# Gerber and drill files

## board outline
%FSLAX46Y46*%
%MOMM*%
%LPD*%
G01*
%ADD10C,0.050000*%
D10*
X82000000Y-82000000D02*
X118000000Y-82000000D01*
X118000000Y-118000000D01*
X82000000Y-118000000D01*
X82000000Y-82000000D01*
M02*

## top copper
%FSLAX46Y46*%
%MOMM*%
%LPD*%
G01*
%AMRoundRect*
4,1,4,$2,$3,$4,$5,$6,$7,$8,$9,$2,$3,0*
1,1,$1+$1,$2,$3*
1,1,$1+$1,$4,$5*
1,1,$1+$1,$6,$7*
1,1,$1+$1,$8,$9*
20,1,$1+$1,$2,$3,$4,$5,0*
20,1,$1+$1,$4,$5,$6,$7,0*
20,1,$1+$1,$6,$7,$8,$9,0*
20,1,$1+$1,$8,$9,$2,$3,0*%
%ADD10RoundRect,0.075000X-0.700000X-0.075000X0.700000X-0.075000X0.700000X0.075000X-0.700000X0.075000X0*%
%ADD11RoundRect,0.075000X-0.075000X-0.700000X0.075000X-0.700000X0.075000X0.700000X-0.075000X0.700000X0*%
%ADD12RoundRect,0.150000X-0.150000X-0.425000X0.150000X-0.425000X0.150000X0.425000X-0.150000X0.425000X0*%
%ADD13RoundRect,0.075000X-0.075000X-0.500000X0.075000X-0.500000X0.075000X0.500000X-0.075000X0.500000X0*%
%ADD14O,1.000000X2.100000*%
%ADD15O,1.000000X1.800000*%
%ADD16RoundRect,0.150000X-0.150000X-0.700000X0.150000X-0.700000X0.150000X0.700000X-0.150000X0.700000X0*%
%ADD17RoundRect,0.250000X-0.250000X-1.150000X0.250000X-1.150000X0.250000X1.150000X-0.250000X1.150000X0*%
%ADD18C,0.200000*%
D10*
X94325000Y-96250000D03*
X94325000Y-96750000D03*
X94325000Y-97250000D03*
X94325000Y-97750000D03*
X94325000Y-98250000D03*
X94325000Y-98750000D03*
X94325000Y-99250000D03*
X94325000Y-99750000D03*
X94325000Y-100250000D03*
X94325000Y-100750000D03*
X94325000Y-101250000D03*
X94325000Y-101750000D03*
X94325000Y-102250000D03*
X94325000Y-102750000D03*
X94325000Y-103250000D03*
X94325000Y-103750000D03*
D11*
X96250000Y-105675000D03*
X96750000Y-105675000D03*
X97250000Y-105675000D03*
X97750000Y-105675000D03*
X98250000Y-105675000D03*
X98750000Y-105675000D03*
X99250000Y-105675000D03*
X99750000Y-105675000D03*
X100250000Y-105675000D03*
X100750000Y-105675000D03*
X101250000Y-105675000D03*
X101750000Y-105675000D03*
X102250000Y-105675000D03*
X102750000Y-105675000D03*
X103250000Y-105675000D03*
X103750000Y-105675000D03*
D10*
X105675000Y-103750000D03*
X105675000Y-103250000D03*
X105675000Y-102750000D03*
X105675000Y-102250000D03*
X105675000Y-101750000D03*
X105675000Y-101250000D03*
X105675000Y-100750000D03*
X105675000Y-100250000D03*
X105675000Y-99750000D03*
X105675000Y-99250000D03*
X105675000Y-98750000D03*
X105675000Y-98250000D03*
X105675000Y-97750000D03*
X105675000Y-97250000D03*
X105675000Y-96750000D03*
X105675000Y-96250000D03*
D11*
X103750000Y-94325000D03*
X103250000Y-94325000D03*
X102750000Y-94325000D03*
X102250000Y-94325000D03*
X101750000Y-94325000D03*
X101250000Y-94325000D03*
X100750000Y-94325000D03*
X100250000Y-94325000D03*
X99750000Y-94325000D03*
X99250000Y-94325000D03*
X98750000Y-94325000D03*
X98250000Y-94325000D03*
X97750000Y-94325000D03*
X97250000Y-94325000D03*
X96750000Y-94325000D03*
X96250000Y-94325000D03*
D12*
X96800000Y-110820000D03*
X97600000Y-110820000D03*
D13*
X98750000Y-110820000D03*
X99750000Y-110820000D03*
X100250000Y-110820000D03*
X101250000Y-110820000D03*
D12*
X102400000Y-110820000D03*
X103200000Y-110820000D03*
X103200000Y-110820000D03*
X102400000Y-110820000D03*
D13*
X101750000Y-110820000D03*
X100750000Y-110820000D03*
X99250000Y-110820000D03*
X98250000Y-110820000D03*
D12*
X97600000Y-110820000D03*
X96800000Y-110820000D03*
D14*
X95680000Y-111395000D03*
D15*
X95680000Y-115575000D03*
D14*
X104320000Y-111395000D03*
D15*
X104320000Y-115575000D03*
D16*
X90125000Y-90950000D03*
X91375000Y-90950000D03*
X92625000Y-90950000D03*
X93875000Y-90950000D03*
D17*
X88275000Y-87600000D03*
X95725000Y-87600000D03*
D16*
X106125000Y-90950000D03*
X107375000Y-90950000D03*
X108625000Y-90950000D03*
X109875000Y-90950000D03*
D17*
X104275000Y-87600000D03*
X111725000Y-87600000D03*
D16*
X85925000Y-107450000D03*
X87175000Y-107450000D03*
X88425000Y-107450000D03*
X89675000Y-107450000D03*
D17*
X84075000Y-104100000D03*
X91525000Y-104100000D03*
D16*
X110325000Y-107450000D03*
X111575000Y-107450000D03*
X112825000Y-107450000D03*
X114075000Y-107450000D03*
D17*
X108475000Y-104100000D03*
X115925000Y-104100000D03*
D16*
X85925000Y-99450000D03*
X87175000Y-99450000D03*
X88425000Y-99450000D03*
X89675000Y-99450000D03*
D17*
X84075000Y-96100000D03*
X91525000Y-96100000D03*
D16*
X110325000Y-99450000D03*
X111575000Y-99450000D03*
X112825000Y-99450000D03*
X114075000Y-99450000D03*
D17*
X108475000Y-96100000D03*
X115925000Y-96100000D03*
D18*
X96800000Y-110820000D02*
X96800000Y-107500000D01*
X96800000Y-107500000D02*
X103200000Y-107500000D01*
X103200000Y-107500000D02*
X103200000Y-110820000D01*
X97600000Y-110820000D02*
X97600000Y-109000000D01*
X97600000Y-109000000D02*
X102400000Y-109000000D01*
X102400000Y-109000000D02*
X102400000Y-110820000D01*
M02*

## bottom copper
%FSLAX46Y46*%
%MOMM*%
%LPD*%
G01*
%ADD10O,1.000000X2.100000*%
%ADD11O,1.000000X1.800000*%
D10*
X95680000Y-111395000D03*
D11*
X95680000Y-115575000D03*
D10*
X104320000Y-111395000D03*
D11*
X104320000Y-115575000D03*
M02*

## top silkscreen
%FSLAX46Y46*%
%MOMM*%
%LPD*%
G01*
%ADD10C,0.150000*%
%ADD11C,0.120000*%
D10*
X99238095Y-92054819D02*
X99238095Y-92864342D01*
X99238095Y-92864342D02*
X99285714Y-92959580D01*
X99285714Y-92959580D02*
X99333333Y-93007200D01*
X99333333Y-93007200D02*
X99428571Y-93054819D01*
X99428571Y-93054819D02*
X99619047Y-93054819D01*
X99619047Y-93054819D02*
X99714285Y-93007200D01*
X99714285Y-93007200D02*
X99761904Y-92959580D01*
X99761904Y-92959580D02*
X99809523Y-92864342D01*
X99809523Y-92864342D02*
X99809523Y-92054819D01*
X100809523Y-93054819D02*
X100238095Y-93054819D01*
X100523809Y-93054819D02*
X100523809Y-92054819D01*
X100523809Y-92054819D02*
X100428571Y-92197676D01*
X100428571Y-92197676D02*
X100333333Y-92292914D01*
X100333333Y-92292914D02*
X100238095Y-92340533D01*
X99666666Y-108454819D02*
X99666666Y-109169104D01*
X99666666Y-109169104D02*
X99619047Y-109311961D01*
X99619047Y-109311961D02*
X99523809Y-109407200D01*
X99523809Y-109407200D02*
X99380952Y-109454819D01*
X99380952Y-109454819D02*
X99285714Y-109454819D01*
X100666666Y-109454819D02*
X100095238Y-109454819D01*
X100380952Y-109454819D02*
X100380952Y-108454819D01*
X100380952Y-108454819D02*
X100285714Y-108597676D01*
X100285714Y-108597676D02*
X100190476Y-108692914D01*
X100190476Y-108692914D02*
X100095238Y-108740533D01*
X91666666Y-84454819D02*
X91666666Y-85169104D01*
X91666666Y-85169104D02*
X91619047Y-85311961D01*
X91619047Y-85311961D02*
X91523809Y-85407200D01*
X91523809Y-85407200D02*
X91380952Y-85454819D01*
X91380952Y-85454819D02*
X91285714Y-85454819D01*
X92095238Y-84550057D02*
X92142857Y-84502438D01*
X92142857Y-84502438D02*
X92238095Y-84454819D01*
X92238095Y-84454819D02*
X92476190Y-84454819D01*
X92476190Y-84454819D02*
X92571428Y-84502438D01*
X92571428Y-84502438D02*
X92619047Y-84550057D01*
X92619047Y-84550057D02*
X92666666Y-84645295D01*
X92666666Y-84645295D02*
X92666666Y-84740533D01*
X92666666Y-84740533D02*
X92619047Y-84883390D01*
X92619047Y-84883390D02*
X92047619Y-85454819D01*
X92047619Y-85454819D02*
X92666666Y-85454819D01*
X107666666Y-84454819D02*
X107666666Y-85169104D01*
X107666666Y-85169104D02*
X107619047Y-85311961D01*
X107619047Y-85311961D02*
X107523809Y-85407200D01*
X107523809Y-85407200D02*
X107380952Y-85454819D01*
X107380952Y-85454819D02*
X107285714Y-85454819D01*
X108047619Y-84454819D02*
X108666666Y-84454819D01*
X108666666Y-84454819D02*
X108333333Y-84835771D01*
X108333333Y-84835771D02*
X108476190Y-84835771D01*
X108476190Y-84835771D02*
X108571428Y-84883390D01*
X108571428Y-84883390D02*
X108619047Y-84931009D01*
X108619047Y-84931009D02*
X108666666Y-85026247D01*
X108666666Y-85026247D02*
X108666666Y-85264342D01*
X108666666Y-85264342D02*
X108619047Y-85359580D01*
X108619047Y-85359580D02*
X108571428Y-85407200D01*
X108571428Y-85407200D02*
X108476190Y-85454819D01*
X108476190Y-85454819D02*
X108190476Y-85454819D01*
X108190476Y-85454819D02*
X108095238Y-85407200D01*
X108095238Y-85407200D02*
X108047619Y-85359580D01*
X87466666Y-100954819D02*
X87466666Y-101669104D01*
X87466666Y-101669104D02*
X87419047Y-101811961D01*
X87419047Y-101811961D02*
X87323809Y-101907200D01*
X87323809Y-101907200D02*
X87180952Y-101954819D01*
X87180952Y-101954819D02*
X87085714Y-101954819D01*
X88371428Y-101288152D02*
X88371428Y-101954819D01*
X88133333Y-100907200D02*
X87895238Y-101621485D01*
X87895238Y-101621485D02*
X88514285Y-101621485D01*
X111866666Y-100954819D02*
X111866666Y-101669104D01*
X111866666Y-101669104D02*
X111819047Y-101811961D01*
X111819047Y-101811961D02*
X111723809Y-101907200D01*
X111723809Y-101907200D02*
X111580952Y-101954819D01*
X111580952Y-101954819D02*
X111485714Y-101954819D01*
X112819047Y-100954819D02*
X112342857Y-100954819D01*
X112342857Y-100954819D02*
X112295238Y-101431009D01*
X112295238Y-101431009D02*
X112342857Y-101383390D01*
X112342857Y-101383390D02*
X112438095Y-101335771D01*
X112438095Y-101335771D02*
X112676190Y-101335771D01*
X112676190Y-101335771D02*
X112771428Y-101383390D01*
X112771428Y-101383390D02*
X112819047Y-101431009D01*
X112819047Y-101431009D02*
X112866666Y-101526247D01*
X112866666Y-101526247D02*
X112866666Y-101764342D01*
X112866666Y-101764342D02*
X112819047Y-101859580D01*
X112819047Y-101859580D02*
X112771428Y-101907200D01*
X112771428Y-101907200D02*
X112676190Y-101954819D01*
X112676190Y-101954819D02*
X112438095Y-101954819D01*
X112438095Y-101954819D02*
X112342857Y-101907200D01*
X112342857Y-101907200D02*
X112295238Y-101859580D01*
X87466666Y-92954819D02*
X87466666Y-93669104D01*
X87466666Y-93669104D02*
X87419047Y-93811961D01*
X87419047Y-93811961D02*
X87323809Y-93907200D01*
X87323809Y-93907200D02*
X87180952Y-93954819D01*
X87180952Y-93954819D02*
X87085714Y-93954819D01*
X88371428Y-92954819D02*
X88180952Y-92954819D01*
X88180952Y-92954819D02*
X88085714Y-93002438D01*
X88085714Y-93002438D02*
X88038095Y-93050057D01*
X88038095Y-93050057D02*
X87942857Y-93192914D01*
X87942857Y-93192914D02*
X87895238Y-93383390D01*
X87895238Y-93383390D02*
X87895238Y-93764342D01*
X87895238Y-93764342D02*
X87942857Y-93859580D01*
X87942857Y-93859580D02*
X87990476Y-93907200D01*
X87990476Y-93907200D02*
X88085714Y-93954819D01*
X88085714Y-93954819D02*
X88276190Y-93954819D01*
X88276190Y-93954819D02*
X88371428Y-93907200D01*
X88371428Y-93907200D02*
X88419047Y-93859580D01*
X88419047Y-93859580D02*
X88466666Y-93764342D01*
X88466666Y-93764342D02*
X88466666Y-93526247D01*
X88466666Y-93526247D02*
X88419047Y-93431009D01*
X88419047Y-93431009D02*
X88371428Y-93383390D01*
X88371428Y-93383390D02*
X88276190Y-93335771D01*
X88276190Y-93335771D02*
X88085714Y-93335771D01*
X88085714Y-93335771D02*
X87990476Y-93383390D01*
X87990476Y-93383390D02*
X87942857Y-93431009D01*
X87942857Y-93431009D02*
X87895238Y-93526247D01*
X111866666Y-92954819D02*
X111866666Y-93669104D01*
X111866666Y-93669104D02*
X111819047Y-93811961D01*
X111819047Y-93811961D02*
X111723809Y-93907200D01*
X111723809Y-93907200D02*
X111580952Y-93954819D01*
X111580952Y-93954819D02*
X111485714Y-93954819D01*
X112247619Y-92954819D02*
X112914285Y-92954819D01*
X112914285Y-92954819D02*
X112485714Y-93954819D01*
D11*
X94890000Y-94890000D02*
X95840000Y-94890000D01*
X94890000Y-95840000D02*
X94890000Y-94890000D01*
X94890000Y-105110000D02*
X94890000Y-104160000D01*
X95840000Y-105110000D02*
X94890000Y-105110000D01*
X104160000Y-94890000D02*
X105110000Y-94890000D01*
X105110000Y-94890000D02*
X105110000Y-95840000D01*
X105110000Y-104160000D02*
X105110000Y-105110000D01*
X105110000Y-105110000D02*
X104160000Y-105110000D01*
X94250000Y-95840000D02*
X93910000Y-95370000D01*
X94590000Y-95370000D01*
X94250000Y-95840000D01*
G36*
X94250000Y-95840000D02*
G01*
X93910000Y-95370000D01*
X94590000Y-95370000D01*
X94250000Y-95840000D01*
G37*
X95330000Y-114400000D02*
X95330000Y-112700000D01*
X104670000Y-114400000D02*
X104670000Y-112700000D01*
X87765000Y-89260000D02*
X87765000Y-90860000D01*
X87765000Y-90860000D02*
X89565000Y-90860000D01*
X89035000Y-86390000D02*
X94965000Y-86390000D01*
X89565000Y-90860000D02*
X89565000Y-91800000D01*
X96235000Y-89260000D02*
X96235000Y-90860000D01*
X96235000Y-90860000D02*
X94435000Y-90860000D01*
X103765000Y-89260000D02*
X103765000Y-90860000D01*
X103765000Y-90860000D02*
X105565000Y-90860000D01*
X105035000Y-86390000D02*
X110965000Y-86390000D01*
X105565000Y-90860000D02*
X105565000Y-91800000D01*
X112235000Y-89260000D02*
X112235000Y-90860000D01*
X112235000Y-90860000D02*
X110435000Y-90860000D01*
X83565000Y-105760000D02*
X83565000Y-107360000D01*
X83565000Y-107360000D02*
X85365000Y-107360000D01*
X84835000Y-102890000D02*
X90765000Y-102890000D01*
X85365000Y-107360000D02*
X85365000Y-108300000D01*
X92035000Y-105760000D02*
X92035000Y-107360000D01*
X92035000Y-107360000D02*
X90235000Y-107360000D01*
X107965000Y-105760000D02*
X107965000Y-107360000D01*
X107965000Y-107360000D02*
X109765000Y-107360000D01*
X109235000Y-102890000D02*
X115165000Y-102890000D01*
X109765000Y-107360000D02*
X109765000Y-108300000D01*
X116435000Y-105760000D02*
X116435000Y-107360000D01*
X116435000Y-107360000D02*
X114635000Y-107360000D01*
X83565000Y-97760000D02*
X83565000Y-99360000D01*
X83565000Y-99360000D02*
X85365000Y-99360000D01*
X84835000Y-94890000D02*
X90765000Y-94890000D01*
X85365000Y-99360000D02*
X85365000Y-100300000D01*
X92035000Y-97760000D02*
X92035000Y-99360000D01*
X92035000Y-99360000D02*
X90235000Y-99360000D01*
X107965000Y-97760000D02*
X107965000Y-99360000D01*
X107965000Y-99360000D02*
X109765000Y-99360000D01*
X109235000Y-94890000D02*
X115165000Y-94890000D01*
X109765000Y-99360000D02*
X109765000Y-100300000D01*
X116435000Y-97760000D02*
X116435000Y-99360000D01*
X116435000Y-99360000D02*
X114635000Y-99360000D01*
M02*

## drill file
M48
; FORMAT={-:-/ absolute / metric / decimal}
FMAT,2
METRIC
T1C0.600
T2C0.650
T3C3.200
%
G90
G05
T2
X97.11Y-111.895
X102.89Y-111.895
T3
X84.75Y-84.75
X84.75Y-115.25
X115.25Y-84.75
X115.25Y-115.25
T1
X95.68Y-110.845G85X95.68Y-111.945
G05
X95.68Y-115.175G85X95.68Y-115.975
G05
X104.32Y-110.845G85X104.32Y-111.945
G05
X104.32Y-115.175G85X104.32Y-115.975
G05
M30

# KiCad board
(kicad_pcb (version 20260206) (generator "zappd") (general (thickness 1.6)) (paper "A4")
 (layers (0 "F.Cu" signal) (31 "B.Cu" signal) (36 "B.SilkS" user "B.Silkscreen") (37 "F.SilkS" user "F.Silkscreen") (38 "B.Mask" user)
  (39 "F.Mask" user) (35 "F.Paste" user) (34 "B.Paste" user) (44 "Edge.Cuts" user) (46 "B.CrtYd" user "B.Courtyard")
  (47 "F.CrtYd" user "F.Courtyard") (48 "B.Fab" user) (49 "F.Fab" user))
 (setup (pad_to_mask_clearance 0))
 (gr_rect (start 82.0 82.0) (end 118.0 118.0) (stroke (width 0.05) (type default)) (fill none) (layer "Edge.Cuts"))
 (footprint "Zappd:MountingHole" (layer "F.Cu") (at 84.75 84.75)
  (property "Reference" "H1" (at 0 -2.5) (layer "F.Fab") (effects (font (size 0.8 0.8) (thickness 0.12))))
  (pad "" np_thru_hole circle (at 0 0) (size 3.2 3.2) (drill 3.2) (layers "*.Cu" "*.Mask")))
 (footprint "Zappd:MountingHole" (layer "F.Cu") (at 115.25 84.75)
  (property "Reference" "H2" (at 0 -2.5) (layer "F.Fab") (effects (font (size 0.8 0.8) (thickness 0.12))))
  (pad "" np_thru_hole circle (at 0 0) (size 3.2 3.2) (drill 3.2) (layers "*.Cu" "*.Mask")))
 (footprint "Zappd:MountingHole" (layer "F.Cu") (at 115.25 115.25)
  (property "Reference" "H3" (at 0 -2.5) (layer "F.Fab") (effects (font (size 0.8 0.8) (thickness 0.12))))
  (pad "" np_thru_hole circle (at 0 0) (size 3.2 3.2) (drill 3.2) (layers "*.Cu" "*.Mask")))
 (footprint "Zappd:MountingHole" (layer "F.Cu") (at 84.75 115.25)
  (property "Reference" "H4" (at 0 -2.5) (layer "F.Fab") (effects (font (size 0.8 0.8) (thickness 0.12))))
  (pad "" np_thru_hole circle (at 0 0) (size 3.2 3.2) (drill 3.2) (layers "*.Cu" "*.Mask")))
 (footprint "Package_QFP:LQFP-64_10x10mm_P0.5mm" (layer "F.Cu") (at 100 100)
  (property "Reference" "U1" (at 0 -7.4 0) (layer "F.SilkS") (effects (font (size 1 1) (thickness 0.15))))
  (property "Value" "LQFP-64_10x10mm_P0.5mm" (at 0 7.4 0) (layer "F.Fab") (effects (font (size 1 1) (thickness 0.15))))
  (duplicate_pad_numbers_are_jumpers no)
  (fp_line (start -5.11 -5.11) (end -4.16 -5.11) (stroke (width 0.12) (type solid)) (layer "F.SilkS"))
  (fp_line (start -5.11 -4.16) (end -5.11 -5.11) (stroke (width 0.12) (type solid)) (layer "F.SilkS"))
  (fp_line (start -5.11 5.11) (end -5.11 4.16) (stroke (width 0.12) (type solid)) (layer "F.SilkS"))
  (fp_line (start -4.16 5.11) (end -5.11 5.11) (stroke (width 0.12) (type solid)) (layer "F.SilkS"))
  (fp_line (start 4.16 -5.11) (end 5.11 -5.11) (stroke (width 0.12) (type solid)) (layer "F.SilkS"))
  (fp_line (start 5.11 -5.11) (end 5.11 -4.16) (stroke (width 0.12) (type solid)) (layer "F.SilkS"))
  (fp_line (start 5.11 4.16) (end 5.11 5.11) (stroke (width 0.12) (type solid)) (layer "F.SilkS"))
  (fp_line (start 5.11 5.11) (end 4.16 5.11) (stroke (width 0.12) (type solid)) (layer "F.SilkS"))
  (fp_poly (pts (xy -5.75 -4.16) (xy -6.09 -4.63) (xy -5.41 -4.63)) (stroke (width 0.12) (type solid)) (fill yes) (layer "F.SilkS"))
  (pad "1" smd roundrect (at -5.675 -3.75) (size 1.55 0.3) (layers "F.Cu" "F.Mask" "F.Paste") (roundrect_rratio 0.25))
  (pad "2" smd roundrect (at -5.675 -3.25) (size 1.55 0.3) (layers "F.Cu" "F.Mask" "F.Paste") (roundrect_rratio 0.25))
  (pad "3" smd roundrect (at -5.675 -2.75) (size 1.55 0.3) (layers "F.Cu" "F.Mask" "F.Paste") (roundrect_rratio 0.25))
  (pad "4" smd roundrect (at -5.675 -2.25) (size 1.55 0.3) (layers "F.Cu" "F.Mask" "F.Paste") (roundrect_rratio 0.25))
  (pad "5" smd roundrect (at -5.675 -1.75) (size 1.55 0.3) (layers "F.Cu" "F.Mask" "F.Paste") (roundrect_rratio 0.25))
  (pad "6" smd roundrect (at -5.675 -1.25) (size 1.55 0.3) (layers "F.Cu" "F.Mask" "F.Paste") (roundrect_rratio 0.25))
  (pad "7" smd roundrect (at -5.675 -0.75) (size 1.55 0.3) (layers "F.Cu" "F.Mask" "F.Paste") (roundrect_rratio 0.25))
  (pad "8" smd roundrect (at -5.675 -0.25) (size 1.55 0.3) (layers "F.Cu" "F.Mask" "F.Paste") (roundrect_rratio 0.25))
  (pad "9" smd roundrect (at -5.675 0.25) (size 1.55 0.3) (layers "F.Cu" "F.Mask" "F.Paste") (roundrect_rratio 0.25))
  (pad "10" smd roundrect (at -5.675 0.75) (size 1.55 0.3) (layers "F.Cu" "F.Mask" "F.Paste") (roundrect_rratio 0.25))
  (pad "11" smd roundrect (at -5.675 1.25) (size 1.55 0.3) (layers "F.Cu" "F.Mask" "F.Paste") (roundrect_rratio 0.25))
  (pad "12" smd roundrect (at -5.675 1.75) (size 1.55 0.3) (layers "F.Cu" "F.Mask" "F.Paste") (roundrect_rratio 0.25))
  (pad "13" smd roundrect (at -5.675 2.25) (size 1.55 0.3) (layers "F.Cu" "F.Mask" "F.Paste") (roundrect_rratio 0.25))
  (pad "14" smd roundrect (at -5.675 2.75) (size 1.55 0.3) (layers "F.Cu" "F.Mask" "F.Paste") (roundrect_rratio 0.25))
  (pad "15" smd roundrect (at -5.675 3.25) (size 1.55 0.3) (layers "F.Cu" "F.Mask" "F.Paste") (roundrect_rratio 0.25))
  (pad "16" smd roundrect (at -5.675 3.75) (size 1.55 0.3) (layers "F.Cu" "F.Mask" "F.Paste") (roundrect_rratio 0.25))
  (pad "17" smd roundrect (at -3.75 5.675) (size 0.3 1.55) (layers "F.Cu" "F.Mask" "F.Paste") (roundrect_rratio 0.25))
  (pad "18" smd roundrect (at -3.25 5.675) (size 0.3 1.55) (layers "F.Cu" "F.Mask" "F.Paste") (roundrect_rratio 0.25))
  (pad "19" smd roundrect (at -2.75 5.675) (size 0.3 1.55) (layers "F.Cu" "F.Mask" "F.Paste") (roundrect_rratio 0.25))
  (pad "20" smd roundrect (at -2.25 5.675) (size 0.3 1.55) (layers "F.Cu" "F.Mask" "F.Paste") (roundrect_rratio 0.25))
  (pad "21" smd roundrect (at -1.75 5.675) (size 0.3 1.55) (layers "F.Cu" "F.Mask" "F.Paste") (roundrect_rratio 0.25))
  (pad "22" smd roundrect (at -1.25 5.675) (size 0.3 1.55) (layers "F.Cu" "F.Mask" "F.Paste") (roundrect_rratio 0.25))
  (pad "23" smd roundrect (at -0.75 5.675) (size 0.3 1.55) (layers "F.Cu" "F.Mask" "F.Paste") (roundrect_rratio 0.25))
  (pad "24" smd roundrect (at -0.25 5.675) (size 0.3 1.55) (layers "F.Cu" "F.Mask" "F.Paste") (roundrect_rratio 0.25))
  (pad "25" smd roundrect (at 0.25 5.675) (size 0.3 1.55) (layers "F.Cu" "F.Mask" "F.Paste") (roundrect_rratio 0.25))
  (pad "26" smd roundrect (at 0.75 5.675) (size 0.3 1.55) (layers "F.Cu" "F.Mask" "F.Paste") (roundrect_rratio 0.25))
  (pad "27" smd roundrect (at 1.25 5.675) (size 0.3 1.55) (layers "F.Cu" "F.Mask" "F.Paste") (roundrect_rratio 0.25))
  (pad "28" smd roundrect (at 1.75 5.675) (size 0.3 1.55) (layers "F.Cu" "F.Mask" "F.Paste") (roundrect_rratio 0.25))
  (pad "29" smd roundrect (at 2.25 5.675) (size 0.3 1.55) (layers "F.Cu" "F.Mask" "F.Paste") (roundrect_rratio 0.25))
  (pad "30" smd roundrect (at 2.75 5.675) (size 0.3 1.55) (layers "F.Cu" "F.Mask" "F.Paste") (roundrect_rratio 0.25))
  (pad "31" smd roundrect (at 3.25 5.675) (size 0.3 1.55) (layers "F.Cu" "F.Mask" "F.Paste") (roundrect_rratio 0.25))
  (pad "32" smd roundrect (at 3.75 5.675) (size 0.3 1.55) (layers "F.Cu" "F.Mask" "F.Paste") (roundrect_rratio 0.25))
  (pad "33" smd roundrect (at 5.675 3.75) (size 1.55 0.3) (layers "F.Cu" "F.Mask" "F.Paste") (roundrect_rratio 0.25))
  (pad "34" smd roundrect (at 5.675 3.25) (size 1.55 0.3) (layers "F.Cu" "F.Mask" "F.Paste") (roundrect_rratio 0.25))
  (pad "35" smd roundrect (at 5.675 2.75) (size 1.55 0.3) (layers "F.Cu" "F.Mask" "F.Paste") (roundrect_rratio 0.25))
  (pad "36" smd roundrect (at 5.675 2.25) (size 1.55 0.3) (layers "F.Cu" "F.Mask" "F.Paste") (roundrect_rratio 0.25))
  (pad "37" smd roundrect (at 5.675 1.75) (size 1.55 0.3) (layers "F.Cu" "F.Mask" "F.Paste") (roundrect_rratio 0.25))
  (pad "38" smd roundrect (at 5.675 1.25) (size 1.55 0.3) (layers "F.Cu" "F.Mask" "F.Paste") (roundrect_rratio 0.25))
  (pad "39" smd roundrect (at 5.675 0.75) (size 1.55 0.3) (layers "F.Cu" "F.Mask" "F.Paste") (roundrect_rratio 0.25))
  (pad "40" smd roundrect (at 5.675 0.25) (size 1.55 0.3) (layers "F.Cu" "F.Mask" "F.Paste") (roundrect_rratio 0.25))
  (pad "41" smd roundrect (at 5.675 -0.25) (size 1.55 0.3) (layers "F.Cu" "F.Mask" "F.Paste") (roundrect_rratio 0.25))
  (pad "42" smd roundrect (at 5.675 -0.75) (size 1.55 0.3) (layers "F.Cu" "F.Mask" "F.Paste") (roundrect_rratio 0.25))
  (pad "43" smd roundrect (at 5.675 -1.25) (size 1.55 0.3) (layers "F.Cu" "F.Mask" "F.Paste") (roundrect_rratio 0.25))
  (pad "44" smd roundrect (at 5.675 -1.75) (size 1.55 0.3) (layers "F.Cu" "F.Mask" "F.Paste") (roundrect_rratio 0.25))
  (pad "45" smd roundrect (at 5.675 -2.25) (size 1.55 0.3) (layers "F.Cu" "F.Mask" "F.Paste") (roundrect_rratio 0.25))
  (pad "46" smd roundrect (at 5.675 -2.75) (size 1.55 0.3) (layers "F.Cu" "F.Mask" "F.Paste") (roundrect_rratio 0.25))
  (pad "47" smd roundrect (at 5.675 -3.25) (size 1.55 0.3) (layers "F.Cu" "F.Mask" "F.Paste") (roundrect_rratio 0.25))
  (pad "48" smd roundrect (at 5.675 -3.75) (size 1.55 0.3) (layers "F.Cu" "F.Mask" "F.Paste") (roundrect_rratio 0.25))
  (pad "49" smd roundrect (at 3.75 -5.675) (size 0.3 1.55) (layers "F.Cu" "F.Mask" "F.Paste") (roundrect_rratio 0.25))
  (pad "50" smd roundrect (at 3.25 -5.675) (size 0.3 1.55) (layers "F.Cu" "F.Mask" "F.Paste") (roundrect_rratio 0.25))
  (pad "51" smd roundrect (at 2.75 -5.675) (size 0.3 1.55) (layers "F.Cu" "F.Mask" "F.Paste") (roundrect_rratio 0.25))
  (pad "52" smd roundrect (at 2.25 -5.675) (size 0.3 1.55) (layers "F.Cu" "F.Mask" "F.Paste") (roundrect_rratio 0.25))
  (pad "53" smd roundrect (at 1.75 -5.675) (size 0.3 1.55) (layers "F.Cu" "F.Mask" "F.Paste") (roundrect_rratio 0.25))
  (pad "54" smd roundrect (at 1.25 -5.675) (size 0.3 1.55) (layers "F.Cu" "F.Mask" "F.Paste") (roundrect_rratio 0.25))
  (pad "55" smd roundrect (at 0.75 -5.675) (size 0.3 1.55) (layers "F.Cu" "F.Mask" "F.Paste") (roundrect_rratio 0.25))
  (pad "56" smd roundrect (at 0.25 -5.675) (size 0.3 1.55) (layers "F.Cu" "F.Mask" "F.Paste") (roundrect_rratio 0.25))
  (pad "57" smd roundrect (at -0.25 -5.675) (size 0.3 1.55) (layers "F.Cu" "F.Mask" "F.Paste") (roundrect_rratio 0.25))
  (pad "58" smd roundrect (at -0.75 -5.675) (size 0.3 1.55) (layers "F.Cu" "F.Mask" "F.Paste") (roundrect_rratio 0.25))
  (pad "59" smd roundrect (at -1.25 -5.675) (size 0.3 1.55) (layers "F.Cu" "F.Mask" "F.Paste") (roundrect_rratio 0.25))
  (pad "60" smd roundrect (at -1.75 -5.675) (size 0.3 1.55) (layers "F.Cu" "F.Mask" "F.Paste") (roundrect_rratio 0.25))
  (pad "61" smd roundrect (at -2.25 -5.675) (size 0.3 1.55) (layers "F.Cu" "F.Mask" "F.Paste") (roundrect_rratio 0.25))
  (pad "62" smd roundrect (at -2.75 -5.675) (size 0.3 1.55) (layers "F.Cu" "F.Mask" "F.Paste") (roundrect_rratio 0.25))
  (pad "63" smd roundrect (at -3.25 -5.675) (size 0.3 1.55) (layers "F.Cu" "F.Mask" "F.Paste") (roundrect_rratio 0.25))
  (pad "64" smd roundrect (at -3.75 -5.675) (size 0.3 1.55) (layers "F.Cu" "F.Mask" "F.Paste") (roundrect_rratio 0.25)))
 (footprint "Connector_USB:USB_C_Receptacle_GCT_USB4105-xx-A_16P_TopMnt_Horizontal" (layer "F.Cu") (at 100 114.5)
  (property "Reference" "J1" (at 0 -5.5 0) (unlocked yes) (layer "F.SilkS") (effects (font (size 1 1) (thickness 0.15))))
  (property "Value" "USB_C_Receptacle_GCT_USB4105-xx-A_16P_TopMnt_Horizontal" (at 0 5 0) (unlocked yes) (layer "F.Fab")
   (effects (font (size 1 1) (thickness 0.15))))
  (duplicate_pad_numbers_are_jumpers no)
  (fp_line (start -4.67 -0.1) (end -4.67 -1.8) (stroke (width 0.12) (type solid)) (layer "F.SilkS"))
  (fp_line (start 4.67 -0.1) (end 4.67 -1.8) (stroke (width 0.12) (type solid)) (layer "F.SilkS"))
  (pad "" np_thru_hole circle (at -2.89 -2.605) (size 0.65 0.65) (drill 0.65) (layers "*.Cu" "*.Mask"))
  (pad "" np_thru_hole circle (at 2.89 -2.605) (size 0.65 0.65) (drill 0.65) (layers "*.Cu" "*.Mask"))
  (pad "A1" smd roundrect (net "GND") (at -3.2 -3.68) (size 0.6 1.15) (layers "F.Cu" "F.Mask" "F.Paste") (roundrect_rratio 0.25))
  (pad "A4" smd roundrect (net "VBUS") (at -2.4 -3.68) (size 0.6 1.15) (layers "F.Cu" "F.Mask" "F.Paste") (roundrect_rratio 0.25))
  (pad "A5" smd roundrect (at -1.25 -3.68) (size 0.3 1.15) (layers "F.Cu" "F.Mask" "F.Paste") (roundrect_rratio 0.25))
  (pad "A6" smd roundrect (at -0.25 -3.68) (size 0.3 1.15) (layers "F.Cu" "F.Mask" "F.Paste") (roundrect_rratio 0.25))
  (pad "A7" smd roundrect (at 0.25 -3.68) (size 0.3 1.15) (layers "F.Cu" "F.Mask" "F.Paste") (roundrect_rratio 0.25))
  (pad "A8" smd roundrect (at 1.25 -3.68) (size 0.3 1.15) (layers "F.Cu" "F.Mask" "F.Paste") (roundrect_rratio 0.25))
  (pad "A9" smd roundrect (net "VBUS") (at 2.4 -3.68) (size 0.6 1.15) (layers "F.Cu" "F.Mask" "F.Paste") (roundrect_rratio 0.25))
  (pad "A12" smd roundrect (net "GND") (at 3.2 -3.68) (size 0.6 1.15) (layers "F.Cu" "F.Mask" "F.Paste") (roundrect_rratio 0.25))
  (pad "B1" smd roundrect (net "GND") (at 3.2 -3.68) (size 0.6 1.15) (layers "F.Cu" "F.Mask" "F.Paste") (roundrect_rratio 0.25))
  (pad "B4" smd roundrect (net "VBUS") (at 2.4 -3.68) (size 0.6 1.15) (layers "F.Cu" "F.Mask" "F.Paste") (roundrect_rratio 0.25))
  (pad "B5" smd roundrect (at 1.75 -3.68) (size 0.3 1.15) (layers "F.Cu" "F.Mask" "F.Paste") (roundrect_rratio 0.25))
  (pad "B6" smd roundrect (at 0.75 -3.68) (size 0.3 1.15) (layers "F.Cu" "F.Mask" "F.Paste") (roundrect_rratio 0.25))
  (pad "B7" smd roundrect (at -0.75 -3.68) (size 0.3 1.15) (layers "F.Cu" "F.Mask" "F.Paste") (roundrect_rratio 0.25))
  (pad "B8" smd roundrect (at -1.75 -3.68) (size 0.3 1.15) (layers "F.Cu" "F.Mask" "F.Paste") (roundrect_rratio 0.25))
  (pad "B9" smd roundrect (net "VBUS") (at -2.4 -3.68) (size 0.6 1.15) (layers "F.Cu" "F.Mask" "F.Paste") (roundrect_rratio 0.25))
  (pad "B12" smd roundrect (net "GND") (at -3.2 -3.68) (size 0.6 1.15) (layers "F.Cu" "F.Mask" "F.Paste") (roundrect_rratio 0.25))
  (pad "SH" thru_hole oval (at -4.32 -3.105) (size 1 2.1) (drill oval 0.6 1.7) (layers "*.Cu" "*.Mask" "F.Paste") (remove_unused_layers no))
  (pad "SH" thru_hole oval (at -4.32 1.075) (size 1 1.8) (drill oval 0.6 1.4) (layers "*.Cu" "*.Mask" "F.Paste") (remove_unused_layers no))
  (pad "SH" thru_hole oval (at 4.32 -3.105) (size 1 2.1) (drill oval 0.6 1.7) (layers "*.Cu" "*.Mask" "F.Paste") (remove_unused_layers no))
  (pad "SH" thru_hole oval (at 4.32 1.075) (size 1 1.8) (drill oval 0.6 1.4) (layers "*.Cu" "*.Mask" "F.Paste") (remove_unused_layers no)))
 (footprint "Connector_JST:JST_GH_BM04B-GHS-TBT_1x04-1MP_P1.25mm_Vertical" (layer "F.Cu") (at 92 89)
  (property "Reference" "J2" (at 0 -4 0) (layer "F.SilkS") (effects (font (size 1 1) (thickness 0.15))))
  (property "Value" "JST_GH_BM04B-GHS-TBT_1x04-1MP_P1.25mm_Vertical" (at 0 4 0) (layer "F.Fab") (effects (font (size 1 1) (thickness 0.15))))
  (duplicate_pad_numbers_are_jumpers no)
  (fp_line (start -4.235 0.26) (end -4.235 1.86) (stroke (width 0.12) (type solid)) (layer "F.SilkS"))
  (fp_line (start -4.235 1.86) (end -2.435 1.86) (stroke (width 0.12) (type solid)) (layer "F.SilkS"))
  (fp_line (start -2.965 -2.61) (end 2.965 -2.61) (stroke (width 0.12) (type solid)) (layer "F.SilkS"))
  (fp_line (start -2.435 1.86) (end -2.435 2.8) (stroke (width 0.12) (type solid)) (layer "F.SilkS"))
  (fp_line (start 4.235 0.26) (end 4.235 1.86) (stroke (width 0.12) (type solid)) (layer "F.SilkS"))
  (fp_line (start 4.235 1.86) (end 2.435 1.86) (stroke (width 0.12) (type solid)) (layer "F.SilkS"))
  (pad "1" smd roundrect (at -1.875 1.95) (size 0.6 1.7) (layers "F.Cu" "F.Mask" "F.Paste") (roundrect_rratio 0.25))
  (pad "2" smd roundrect (at -0.625 1.95) (size 0.6 1.7) (layers "F.Cu" "F.Mask" "F.Paste") (roundrect_rratio 0.25))
  (pad "3" smd roundrect (at 0.625 1.95) (size 0.6 1.7) (layers "F.Cu" "F.Mask" "F.Paste") (roundrect_rratio 0.25))
  (pad "4" smd roundrect (at 1.875 1.95) (size 0.6 1.7) (layers "F.Cu" "F.Mask" "F.Paste") (roundrect_rratio 0.25))
  (pad "MP" smd roundrect (at -3.725 -1.4) (size 1 2.8) (layers "F.Cu" "F.Mask" "F.Paste") (roundrect_rratio 0.25))
  (pad "MP" smd roundrect (at 3.725 -1.4) (size 1 2.8) (layers "F.Cu" "F.Mask" "F.Paste") (roundrect_rratio 0.25)))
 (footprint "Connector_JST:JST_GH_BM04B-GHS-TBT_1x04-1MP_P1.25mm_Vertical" (layer "F.Cu") (at 108 89)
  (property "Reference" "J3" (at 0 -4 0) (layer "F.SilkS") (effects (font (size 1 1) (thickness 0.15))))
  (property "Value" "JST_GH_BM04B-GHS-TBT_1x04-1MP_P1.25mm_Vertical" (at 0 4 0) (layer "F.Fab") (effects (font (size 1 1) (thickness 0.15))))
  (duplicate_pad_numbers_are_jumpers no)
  (fp_line (start -4.235 0.26) (end -4.235 1.86) (stroke (width 0.12) (type solid)) (layer "F.SilkS"))
  (fp_line (start -4.235 1.86) (end -2.435 1.86) (stroke (width 0.12) (type solid)) (layer "F.SilkS"))
  (fp_line (start -2.965 -2.61) (end 2.965 -2.61) (stroke (width 0.12) (type solid)) (layer "F.SilkS"))
  (fp_line (start -2.435 1.86) (end -2.435 2.8) (stroke (width 0.12) (type solid)) (layer "F.SilkS"))
  (fp_line (start 4.235 0.26) (end 4.235 1.86) (stroke (width 0.12) (type solid)) (layer "F.SilkS"))
  (fp_line (start 4.235 1.86) (end 2.435 1.86) (stroke (width 0.12) (type solid)) (layer "F.SilkS"))
  (pad "1" smd roundrect (at -1.875 1.95) (size 0.6 1.7) (layers "F.Cu" "F.Mask" "F.Paste") (roundrect_rratio 0.25))
  (pad "2" smd roundrect (at -0.625 1.95) (size 0.6 1.7) (layers "F.Cu" "F.Mask" "F.Paste") (roundrect_rratio 0.25))
  (pad "3" smd roundrect (at 0.625 1.95) (size 0.6 1.7) (layers "F.Cu" "F.Mask" "F.Paste") (roundrect_rratio 0.25))
  (pad "4" smd roundrect (at 1.875 1.95) (size 0.6 1.7) (layers "F.Cu" "F.Mask" "F.Paste") (roundrect_rratio 0.25))
  (pad "MP" smd roundrect (at -3.725 -1.4) (size 1 2.8) (layers "F.Cu" "F.Mask" "F.Paste") (roundrect_rratio 0.25))
  (pad "MP" smd roundrect (at 3.725 -1.4) (size 1 2.8) (layers "F.Cu" "F.Mask" "F.Paste") (roundrect_rratio 0.25)))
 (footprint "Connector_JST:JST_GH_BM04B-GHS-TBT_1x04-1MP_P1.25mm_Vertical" (layer "F.Cu") (at 87.8 105.5)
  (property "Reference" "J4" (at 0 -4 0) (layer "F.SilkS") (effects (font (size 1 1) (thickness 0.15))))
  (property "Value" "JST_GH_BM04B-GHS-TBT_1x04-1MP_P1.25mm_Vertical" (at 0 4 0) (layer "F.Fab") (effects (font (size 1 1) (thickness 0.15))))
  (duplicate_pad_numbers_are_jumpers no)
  (fp_line (start -4.235 0.26) (end -4.235 1.86) (stroke (width 0.12) (type solid)) (layer "F.SilkS"))
  (fp_line (start -4.235 1.86) (end -2.435 1.86) (stroke (width 0.12) (type solid)) (layer "F.SilkS"))
  (fp_line (start -2.965 -2.61) (end 2.965 -2.61) (stroke (width 0.12) (type solid)) (layer "F.SilkS"))
  (fp_line (start -2.435 1.86) (end -2.435 2.8) (stroke (width 0.12) (type solid)) (layer "F.SilkS"))
  (fp_line (start 4.235 0.26) (end 4.235 1.86) (stroke (width 0.12) (type solid)) (layer "F.SilkS"))
  (fp_line (start 4.235 1.86) (end 2.435 1.86) (stroke (width 0.12) (type solid)) (layer "F.SilkS"))
  (pad "1" smd roundrect (at -1.875 1.95) (size 0.6 1.7) (layers "F.Cu" "F.Mask" "F.Paste") (roundrect_rratio 0.25))
  (pad "2" smd roundrect (at -0.625 1.95) (size 0.6 1.7) (layers "F.Cu" "F.Mask" "F.Paste") (roundrect_rratio 0.25))
  (pad "3" smd roundrect (at 0.625 1.95) (size 0.6 1.7) (layers "F.Cu" "F.Mask" "F.Paste") (roundrect_rratio 0.25))
  (pad "4" smd roundrect (at 1.875 1.95) (size 0.6 1.7) (layers "F.Cu" "F.Mask" "F.Paste") (roundrect_rratio 0.25))
  (pad "MP" smd roundrect (at -3.725 -1.4) (size 1 2.8) (layers "F.Cu" "F.Mask" "F.Paste") (roundrect_rratio 0.25))
  (pad "MP" smd roundrect (at 3.725 -1.4) (size 1 2.8) (layers "F.Cu" "F.Mask" "F.Paste") (roundrect_rratio 0.25)))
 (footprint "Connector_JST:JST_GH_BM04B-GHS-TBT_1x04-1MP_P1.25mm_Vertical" (layer "F.Cu") (at 112.2 105.5)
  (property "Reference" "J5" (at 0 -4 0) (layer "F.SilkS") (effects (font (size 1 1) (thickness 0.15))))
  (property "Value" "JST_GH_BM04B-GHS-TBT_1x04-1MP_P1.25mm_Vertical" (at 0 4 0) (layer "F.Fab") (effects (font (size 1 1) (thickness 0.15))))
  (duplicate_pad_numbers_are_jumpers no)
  (fp_line (start -4.235 0.26) (end -4.235 1.86) (stroke (width 0.12) (type solid)) (layer "F.SilkS"))
  (fp_line (start -4.235 1.86) (end -2.435 1.86) (stroke (width 0.12) (type solid)) (layer "F.SilkS"))
  (fp_line (start -2.965 -2.61) (end 2.965 -2.61) (stroke (width 0.12) (type solid)) (layer "F.SilkS"))
  (fp_line (start -2.435 1.86) (end -2.435 2.8) (stroke (width 0.12) (type solid)) (layer "F.SilkS"))
  (fp_line (start 4.235 0.26) (end 4.235 1.86) (stroke (width 0.12) (type solid)) (layer "F.SilkS"))
  (fp_line (start 4.235 1.86) (end 2.435 1.86) (stroke (width 0.12) (type solid)) (layer "F.SilkS"))
  (pad "1" smd roundrect (at -1.875 1.95) (size 0.6 1.7) (layers "F.Cu" "F.Mask" "F.Paste") (roundrect_rratio 0.25))
  (pad "2" smd roundrect (at -0.625 1.95) (size 0.6 1.7) (layers "F.Cu" "F.Mask" "F.Paste") (roundrect_rratio 0.25))
  (pad "3" smd roundrect (at 0.625 1.95) (size 0.6 1.7) (layers "F.Cu" "F.Mask" "F.Paste") (roundrect_rratio 0.25))
  (pad "4" smd roundrect (at 1.875 1.95) (size 0.6 1.7) (layers "F.Cu" "F.Mask" "F.Paste") (roundrect_rratio 0.25))
  (pad "MP" smd roundrect (at -3.725 -1.4) (size 1 2.8) (layers "F.Cu" "F.Mask" "F.Paste") (roundrect_rratio 0.25))
  (pad "MP" smd roundrect (at 3.725 -1.4) (size 1 2.8) (layers "F.Cu" "F.Mask" "F.Paste") (roundrect_rratio 0.25)))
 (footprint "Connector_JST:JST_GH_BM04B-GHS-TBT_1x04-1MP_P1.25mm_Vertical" (layer "F.Cu") (at 87.8 97.5)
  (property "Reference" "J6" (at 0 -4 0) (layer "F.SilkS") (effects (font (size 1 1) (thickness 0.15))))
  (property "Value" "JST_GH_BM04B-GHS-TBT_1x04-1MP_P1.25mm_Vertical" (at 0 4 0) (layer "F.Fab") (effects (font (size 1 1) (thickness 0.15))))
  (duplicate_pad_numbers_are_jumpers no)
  (fp_line (start -4.235 0.26) (end -4.235 1.86) (stroke (width 0.12) (type solid)) (layer "F.SilkS"))
  (fp_line (start -4.235 1.86) (end -2.435 1.86) (stroke (width 0.12) (type solid)) (layer "F.SilkS"))
  (fp_line (start -2.965 -2.61) (end 2.965 -2.61) (stroke (width 0.12) (type solid)) (layer "F.SilkS"))
  (fp_line (start -2.435 1.86) (end -2.435 2.8) (stroke (width 0.12) (type solid)) (layer "F.SilkS"))
  (fp_line (start 4.235 0.26) (end 4.235 1.86) (stroke (width 0.12) (type solid)) (layer "F.SilkS"))
  (fp_line (start 4.235 1.86) (end 2.435 1.86) (stroke (width 0.12) (type solid)) (layer "F.SilkS"))
  (pad "1" smd roundrect (at -1.875 1.95) (size 0.6 1.7) (layers "F.Cu" "F.Mask" "F.Paste") (roundrect_rratio 0.25))
  (pad "2" smd roundrect (at -0.625 1.95) (size 0.6 1.7) (layers "F.Cu" "F.Mask" "F.Paste") (roundrect_rratio 0.25))
  (pad "3" smd roundrect (at 0.625 1.95) (size 0.6 1.7) (layers "F.Cu" "F.Mask" "F.Paste") (roundrect_rratio 0.25))
  (pad "4" smd roundrect (at 1.875 1.95) (size 0.6 1.7) (layers "F.Cu" "F.Mask" "F.Paste") (roundrect_rratio 0.25))
  (pad "MP" smd roundrect (at -3.725 -1.4) (size 1 2.8) (layers "F.Cu" "F.Mask" "F.Paste") (roundrect_rratio 0.25))
  (pad "MP" smd roundrect (at 3.725 -1.4) (size 1 2.8) (layers "F.Cu" "F.Mask" "F.Paste") (roundrect_rratio 0.25)))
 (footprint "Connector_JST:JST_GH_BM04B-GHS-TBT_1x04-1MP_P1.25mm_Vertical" (layer "F.Cu") (at 112.2 97.5)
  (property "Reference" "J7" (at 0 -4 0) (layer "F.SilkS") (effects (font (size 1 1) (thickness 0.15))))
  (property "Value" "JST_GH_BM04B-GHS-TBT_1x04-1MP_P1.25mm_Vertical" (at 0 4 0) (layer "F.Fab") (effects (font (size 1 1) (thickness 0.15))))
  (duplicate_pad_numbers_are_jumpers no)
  (fp_line (start -4.235 0.26) (end -4.235 1.86) (stroke (width 0.12) (type solid)) (layer "F.SilkS"))
  (fp_line (start -4.235 1.86) (end -2.435 1.86) (stroke (width 0.12) (type solid)) (layer "F.SilkS"))
  (fp_line (start -2.965 -2.61) (end 2.965 -2.61) (stroke (width 0.12) (type solid)) (layer "F.SilkS"))
  (fp_line (start -2.435 1.86) (end -2.435 2.8) (stroke (width 0.12) (type solid)) (layer "F.SilkS"))
  (fp_line (start 4.235 0.26) (end 4.235 1.86) (stroke (width 0.12) (type solid)) (layer "F.SilkS"))
  (fp_line (start 4.235 1.86) (end 2.435 1.86) (stroke (width 0.12) (type solid)) (layer "F.SilkS"))
  (pad "1" smd roundrect (at -1.875 1.95) (size 0.6 1.7) (layers "F.Cu" "F.Mask" "F.Paste") (roundrect_rratio 0.25))
  (pad "2" smd roundrect (at -0.625 1.95) (size 0.6 1.7) (layers "F.Cu" "F.Mask" "F.Paste") (roundrect_rratio 0.25))
  (pad "3" smd roundrect (at 0.625 1.95) (size 0.6 1.7) (layers "F.Cu" "F.Mask" "F.Paste") (roundrect_rratio 0.25))
  (pad "4" smd roundrect (at 1.875 1.95) (size 0.6 1.7) (layers "F.Cu" "F.Mask" "F.Paste") (roundrect_rratio 0.25))
  (pad "MP" smd roundrect (at -3.725 -1.4) (size 1 2.8) (layers "F.Cu" "F.Mask" "F.Paste") (roundrect_rratio 0.25))
  (pad "MP" smd roundrect (at 3.725 -1.4) (size 1 2.8) (layers "F.Cu" "F.Mask" "F.Paste") (roundrect_rratio 0.25)))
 (segment (start 96.8000 110.8200) (end 96.8000 107.5000) (width 0.2) (layer "F.Cu") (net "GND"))
 (segment (start 96.8000 107.5000) (end 103.2000 107.5000) (width 0.2) (layer "F.Cu") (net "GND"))
 (segment (start 103.2000 107.5000) (end 103.2000 110.8200) (width 0.2) (layer "F.Cu") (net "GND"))
 (segment (start 97.6000 110.8200) (end 97.6000 109.0000) (width 0.2) (layer "F.Cu") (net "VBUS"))
 (segment (start 97.6000 109.0000) (end 102.4000 109.0000) (width 0.2) (layer "F.Cu") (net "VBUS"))
 (segment (start 102.4000 109.0000) (end 102.4000 110.8200) (width 0.2) (layer "F.Cu") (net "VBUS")))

